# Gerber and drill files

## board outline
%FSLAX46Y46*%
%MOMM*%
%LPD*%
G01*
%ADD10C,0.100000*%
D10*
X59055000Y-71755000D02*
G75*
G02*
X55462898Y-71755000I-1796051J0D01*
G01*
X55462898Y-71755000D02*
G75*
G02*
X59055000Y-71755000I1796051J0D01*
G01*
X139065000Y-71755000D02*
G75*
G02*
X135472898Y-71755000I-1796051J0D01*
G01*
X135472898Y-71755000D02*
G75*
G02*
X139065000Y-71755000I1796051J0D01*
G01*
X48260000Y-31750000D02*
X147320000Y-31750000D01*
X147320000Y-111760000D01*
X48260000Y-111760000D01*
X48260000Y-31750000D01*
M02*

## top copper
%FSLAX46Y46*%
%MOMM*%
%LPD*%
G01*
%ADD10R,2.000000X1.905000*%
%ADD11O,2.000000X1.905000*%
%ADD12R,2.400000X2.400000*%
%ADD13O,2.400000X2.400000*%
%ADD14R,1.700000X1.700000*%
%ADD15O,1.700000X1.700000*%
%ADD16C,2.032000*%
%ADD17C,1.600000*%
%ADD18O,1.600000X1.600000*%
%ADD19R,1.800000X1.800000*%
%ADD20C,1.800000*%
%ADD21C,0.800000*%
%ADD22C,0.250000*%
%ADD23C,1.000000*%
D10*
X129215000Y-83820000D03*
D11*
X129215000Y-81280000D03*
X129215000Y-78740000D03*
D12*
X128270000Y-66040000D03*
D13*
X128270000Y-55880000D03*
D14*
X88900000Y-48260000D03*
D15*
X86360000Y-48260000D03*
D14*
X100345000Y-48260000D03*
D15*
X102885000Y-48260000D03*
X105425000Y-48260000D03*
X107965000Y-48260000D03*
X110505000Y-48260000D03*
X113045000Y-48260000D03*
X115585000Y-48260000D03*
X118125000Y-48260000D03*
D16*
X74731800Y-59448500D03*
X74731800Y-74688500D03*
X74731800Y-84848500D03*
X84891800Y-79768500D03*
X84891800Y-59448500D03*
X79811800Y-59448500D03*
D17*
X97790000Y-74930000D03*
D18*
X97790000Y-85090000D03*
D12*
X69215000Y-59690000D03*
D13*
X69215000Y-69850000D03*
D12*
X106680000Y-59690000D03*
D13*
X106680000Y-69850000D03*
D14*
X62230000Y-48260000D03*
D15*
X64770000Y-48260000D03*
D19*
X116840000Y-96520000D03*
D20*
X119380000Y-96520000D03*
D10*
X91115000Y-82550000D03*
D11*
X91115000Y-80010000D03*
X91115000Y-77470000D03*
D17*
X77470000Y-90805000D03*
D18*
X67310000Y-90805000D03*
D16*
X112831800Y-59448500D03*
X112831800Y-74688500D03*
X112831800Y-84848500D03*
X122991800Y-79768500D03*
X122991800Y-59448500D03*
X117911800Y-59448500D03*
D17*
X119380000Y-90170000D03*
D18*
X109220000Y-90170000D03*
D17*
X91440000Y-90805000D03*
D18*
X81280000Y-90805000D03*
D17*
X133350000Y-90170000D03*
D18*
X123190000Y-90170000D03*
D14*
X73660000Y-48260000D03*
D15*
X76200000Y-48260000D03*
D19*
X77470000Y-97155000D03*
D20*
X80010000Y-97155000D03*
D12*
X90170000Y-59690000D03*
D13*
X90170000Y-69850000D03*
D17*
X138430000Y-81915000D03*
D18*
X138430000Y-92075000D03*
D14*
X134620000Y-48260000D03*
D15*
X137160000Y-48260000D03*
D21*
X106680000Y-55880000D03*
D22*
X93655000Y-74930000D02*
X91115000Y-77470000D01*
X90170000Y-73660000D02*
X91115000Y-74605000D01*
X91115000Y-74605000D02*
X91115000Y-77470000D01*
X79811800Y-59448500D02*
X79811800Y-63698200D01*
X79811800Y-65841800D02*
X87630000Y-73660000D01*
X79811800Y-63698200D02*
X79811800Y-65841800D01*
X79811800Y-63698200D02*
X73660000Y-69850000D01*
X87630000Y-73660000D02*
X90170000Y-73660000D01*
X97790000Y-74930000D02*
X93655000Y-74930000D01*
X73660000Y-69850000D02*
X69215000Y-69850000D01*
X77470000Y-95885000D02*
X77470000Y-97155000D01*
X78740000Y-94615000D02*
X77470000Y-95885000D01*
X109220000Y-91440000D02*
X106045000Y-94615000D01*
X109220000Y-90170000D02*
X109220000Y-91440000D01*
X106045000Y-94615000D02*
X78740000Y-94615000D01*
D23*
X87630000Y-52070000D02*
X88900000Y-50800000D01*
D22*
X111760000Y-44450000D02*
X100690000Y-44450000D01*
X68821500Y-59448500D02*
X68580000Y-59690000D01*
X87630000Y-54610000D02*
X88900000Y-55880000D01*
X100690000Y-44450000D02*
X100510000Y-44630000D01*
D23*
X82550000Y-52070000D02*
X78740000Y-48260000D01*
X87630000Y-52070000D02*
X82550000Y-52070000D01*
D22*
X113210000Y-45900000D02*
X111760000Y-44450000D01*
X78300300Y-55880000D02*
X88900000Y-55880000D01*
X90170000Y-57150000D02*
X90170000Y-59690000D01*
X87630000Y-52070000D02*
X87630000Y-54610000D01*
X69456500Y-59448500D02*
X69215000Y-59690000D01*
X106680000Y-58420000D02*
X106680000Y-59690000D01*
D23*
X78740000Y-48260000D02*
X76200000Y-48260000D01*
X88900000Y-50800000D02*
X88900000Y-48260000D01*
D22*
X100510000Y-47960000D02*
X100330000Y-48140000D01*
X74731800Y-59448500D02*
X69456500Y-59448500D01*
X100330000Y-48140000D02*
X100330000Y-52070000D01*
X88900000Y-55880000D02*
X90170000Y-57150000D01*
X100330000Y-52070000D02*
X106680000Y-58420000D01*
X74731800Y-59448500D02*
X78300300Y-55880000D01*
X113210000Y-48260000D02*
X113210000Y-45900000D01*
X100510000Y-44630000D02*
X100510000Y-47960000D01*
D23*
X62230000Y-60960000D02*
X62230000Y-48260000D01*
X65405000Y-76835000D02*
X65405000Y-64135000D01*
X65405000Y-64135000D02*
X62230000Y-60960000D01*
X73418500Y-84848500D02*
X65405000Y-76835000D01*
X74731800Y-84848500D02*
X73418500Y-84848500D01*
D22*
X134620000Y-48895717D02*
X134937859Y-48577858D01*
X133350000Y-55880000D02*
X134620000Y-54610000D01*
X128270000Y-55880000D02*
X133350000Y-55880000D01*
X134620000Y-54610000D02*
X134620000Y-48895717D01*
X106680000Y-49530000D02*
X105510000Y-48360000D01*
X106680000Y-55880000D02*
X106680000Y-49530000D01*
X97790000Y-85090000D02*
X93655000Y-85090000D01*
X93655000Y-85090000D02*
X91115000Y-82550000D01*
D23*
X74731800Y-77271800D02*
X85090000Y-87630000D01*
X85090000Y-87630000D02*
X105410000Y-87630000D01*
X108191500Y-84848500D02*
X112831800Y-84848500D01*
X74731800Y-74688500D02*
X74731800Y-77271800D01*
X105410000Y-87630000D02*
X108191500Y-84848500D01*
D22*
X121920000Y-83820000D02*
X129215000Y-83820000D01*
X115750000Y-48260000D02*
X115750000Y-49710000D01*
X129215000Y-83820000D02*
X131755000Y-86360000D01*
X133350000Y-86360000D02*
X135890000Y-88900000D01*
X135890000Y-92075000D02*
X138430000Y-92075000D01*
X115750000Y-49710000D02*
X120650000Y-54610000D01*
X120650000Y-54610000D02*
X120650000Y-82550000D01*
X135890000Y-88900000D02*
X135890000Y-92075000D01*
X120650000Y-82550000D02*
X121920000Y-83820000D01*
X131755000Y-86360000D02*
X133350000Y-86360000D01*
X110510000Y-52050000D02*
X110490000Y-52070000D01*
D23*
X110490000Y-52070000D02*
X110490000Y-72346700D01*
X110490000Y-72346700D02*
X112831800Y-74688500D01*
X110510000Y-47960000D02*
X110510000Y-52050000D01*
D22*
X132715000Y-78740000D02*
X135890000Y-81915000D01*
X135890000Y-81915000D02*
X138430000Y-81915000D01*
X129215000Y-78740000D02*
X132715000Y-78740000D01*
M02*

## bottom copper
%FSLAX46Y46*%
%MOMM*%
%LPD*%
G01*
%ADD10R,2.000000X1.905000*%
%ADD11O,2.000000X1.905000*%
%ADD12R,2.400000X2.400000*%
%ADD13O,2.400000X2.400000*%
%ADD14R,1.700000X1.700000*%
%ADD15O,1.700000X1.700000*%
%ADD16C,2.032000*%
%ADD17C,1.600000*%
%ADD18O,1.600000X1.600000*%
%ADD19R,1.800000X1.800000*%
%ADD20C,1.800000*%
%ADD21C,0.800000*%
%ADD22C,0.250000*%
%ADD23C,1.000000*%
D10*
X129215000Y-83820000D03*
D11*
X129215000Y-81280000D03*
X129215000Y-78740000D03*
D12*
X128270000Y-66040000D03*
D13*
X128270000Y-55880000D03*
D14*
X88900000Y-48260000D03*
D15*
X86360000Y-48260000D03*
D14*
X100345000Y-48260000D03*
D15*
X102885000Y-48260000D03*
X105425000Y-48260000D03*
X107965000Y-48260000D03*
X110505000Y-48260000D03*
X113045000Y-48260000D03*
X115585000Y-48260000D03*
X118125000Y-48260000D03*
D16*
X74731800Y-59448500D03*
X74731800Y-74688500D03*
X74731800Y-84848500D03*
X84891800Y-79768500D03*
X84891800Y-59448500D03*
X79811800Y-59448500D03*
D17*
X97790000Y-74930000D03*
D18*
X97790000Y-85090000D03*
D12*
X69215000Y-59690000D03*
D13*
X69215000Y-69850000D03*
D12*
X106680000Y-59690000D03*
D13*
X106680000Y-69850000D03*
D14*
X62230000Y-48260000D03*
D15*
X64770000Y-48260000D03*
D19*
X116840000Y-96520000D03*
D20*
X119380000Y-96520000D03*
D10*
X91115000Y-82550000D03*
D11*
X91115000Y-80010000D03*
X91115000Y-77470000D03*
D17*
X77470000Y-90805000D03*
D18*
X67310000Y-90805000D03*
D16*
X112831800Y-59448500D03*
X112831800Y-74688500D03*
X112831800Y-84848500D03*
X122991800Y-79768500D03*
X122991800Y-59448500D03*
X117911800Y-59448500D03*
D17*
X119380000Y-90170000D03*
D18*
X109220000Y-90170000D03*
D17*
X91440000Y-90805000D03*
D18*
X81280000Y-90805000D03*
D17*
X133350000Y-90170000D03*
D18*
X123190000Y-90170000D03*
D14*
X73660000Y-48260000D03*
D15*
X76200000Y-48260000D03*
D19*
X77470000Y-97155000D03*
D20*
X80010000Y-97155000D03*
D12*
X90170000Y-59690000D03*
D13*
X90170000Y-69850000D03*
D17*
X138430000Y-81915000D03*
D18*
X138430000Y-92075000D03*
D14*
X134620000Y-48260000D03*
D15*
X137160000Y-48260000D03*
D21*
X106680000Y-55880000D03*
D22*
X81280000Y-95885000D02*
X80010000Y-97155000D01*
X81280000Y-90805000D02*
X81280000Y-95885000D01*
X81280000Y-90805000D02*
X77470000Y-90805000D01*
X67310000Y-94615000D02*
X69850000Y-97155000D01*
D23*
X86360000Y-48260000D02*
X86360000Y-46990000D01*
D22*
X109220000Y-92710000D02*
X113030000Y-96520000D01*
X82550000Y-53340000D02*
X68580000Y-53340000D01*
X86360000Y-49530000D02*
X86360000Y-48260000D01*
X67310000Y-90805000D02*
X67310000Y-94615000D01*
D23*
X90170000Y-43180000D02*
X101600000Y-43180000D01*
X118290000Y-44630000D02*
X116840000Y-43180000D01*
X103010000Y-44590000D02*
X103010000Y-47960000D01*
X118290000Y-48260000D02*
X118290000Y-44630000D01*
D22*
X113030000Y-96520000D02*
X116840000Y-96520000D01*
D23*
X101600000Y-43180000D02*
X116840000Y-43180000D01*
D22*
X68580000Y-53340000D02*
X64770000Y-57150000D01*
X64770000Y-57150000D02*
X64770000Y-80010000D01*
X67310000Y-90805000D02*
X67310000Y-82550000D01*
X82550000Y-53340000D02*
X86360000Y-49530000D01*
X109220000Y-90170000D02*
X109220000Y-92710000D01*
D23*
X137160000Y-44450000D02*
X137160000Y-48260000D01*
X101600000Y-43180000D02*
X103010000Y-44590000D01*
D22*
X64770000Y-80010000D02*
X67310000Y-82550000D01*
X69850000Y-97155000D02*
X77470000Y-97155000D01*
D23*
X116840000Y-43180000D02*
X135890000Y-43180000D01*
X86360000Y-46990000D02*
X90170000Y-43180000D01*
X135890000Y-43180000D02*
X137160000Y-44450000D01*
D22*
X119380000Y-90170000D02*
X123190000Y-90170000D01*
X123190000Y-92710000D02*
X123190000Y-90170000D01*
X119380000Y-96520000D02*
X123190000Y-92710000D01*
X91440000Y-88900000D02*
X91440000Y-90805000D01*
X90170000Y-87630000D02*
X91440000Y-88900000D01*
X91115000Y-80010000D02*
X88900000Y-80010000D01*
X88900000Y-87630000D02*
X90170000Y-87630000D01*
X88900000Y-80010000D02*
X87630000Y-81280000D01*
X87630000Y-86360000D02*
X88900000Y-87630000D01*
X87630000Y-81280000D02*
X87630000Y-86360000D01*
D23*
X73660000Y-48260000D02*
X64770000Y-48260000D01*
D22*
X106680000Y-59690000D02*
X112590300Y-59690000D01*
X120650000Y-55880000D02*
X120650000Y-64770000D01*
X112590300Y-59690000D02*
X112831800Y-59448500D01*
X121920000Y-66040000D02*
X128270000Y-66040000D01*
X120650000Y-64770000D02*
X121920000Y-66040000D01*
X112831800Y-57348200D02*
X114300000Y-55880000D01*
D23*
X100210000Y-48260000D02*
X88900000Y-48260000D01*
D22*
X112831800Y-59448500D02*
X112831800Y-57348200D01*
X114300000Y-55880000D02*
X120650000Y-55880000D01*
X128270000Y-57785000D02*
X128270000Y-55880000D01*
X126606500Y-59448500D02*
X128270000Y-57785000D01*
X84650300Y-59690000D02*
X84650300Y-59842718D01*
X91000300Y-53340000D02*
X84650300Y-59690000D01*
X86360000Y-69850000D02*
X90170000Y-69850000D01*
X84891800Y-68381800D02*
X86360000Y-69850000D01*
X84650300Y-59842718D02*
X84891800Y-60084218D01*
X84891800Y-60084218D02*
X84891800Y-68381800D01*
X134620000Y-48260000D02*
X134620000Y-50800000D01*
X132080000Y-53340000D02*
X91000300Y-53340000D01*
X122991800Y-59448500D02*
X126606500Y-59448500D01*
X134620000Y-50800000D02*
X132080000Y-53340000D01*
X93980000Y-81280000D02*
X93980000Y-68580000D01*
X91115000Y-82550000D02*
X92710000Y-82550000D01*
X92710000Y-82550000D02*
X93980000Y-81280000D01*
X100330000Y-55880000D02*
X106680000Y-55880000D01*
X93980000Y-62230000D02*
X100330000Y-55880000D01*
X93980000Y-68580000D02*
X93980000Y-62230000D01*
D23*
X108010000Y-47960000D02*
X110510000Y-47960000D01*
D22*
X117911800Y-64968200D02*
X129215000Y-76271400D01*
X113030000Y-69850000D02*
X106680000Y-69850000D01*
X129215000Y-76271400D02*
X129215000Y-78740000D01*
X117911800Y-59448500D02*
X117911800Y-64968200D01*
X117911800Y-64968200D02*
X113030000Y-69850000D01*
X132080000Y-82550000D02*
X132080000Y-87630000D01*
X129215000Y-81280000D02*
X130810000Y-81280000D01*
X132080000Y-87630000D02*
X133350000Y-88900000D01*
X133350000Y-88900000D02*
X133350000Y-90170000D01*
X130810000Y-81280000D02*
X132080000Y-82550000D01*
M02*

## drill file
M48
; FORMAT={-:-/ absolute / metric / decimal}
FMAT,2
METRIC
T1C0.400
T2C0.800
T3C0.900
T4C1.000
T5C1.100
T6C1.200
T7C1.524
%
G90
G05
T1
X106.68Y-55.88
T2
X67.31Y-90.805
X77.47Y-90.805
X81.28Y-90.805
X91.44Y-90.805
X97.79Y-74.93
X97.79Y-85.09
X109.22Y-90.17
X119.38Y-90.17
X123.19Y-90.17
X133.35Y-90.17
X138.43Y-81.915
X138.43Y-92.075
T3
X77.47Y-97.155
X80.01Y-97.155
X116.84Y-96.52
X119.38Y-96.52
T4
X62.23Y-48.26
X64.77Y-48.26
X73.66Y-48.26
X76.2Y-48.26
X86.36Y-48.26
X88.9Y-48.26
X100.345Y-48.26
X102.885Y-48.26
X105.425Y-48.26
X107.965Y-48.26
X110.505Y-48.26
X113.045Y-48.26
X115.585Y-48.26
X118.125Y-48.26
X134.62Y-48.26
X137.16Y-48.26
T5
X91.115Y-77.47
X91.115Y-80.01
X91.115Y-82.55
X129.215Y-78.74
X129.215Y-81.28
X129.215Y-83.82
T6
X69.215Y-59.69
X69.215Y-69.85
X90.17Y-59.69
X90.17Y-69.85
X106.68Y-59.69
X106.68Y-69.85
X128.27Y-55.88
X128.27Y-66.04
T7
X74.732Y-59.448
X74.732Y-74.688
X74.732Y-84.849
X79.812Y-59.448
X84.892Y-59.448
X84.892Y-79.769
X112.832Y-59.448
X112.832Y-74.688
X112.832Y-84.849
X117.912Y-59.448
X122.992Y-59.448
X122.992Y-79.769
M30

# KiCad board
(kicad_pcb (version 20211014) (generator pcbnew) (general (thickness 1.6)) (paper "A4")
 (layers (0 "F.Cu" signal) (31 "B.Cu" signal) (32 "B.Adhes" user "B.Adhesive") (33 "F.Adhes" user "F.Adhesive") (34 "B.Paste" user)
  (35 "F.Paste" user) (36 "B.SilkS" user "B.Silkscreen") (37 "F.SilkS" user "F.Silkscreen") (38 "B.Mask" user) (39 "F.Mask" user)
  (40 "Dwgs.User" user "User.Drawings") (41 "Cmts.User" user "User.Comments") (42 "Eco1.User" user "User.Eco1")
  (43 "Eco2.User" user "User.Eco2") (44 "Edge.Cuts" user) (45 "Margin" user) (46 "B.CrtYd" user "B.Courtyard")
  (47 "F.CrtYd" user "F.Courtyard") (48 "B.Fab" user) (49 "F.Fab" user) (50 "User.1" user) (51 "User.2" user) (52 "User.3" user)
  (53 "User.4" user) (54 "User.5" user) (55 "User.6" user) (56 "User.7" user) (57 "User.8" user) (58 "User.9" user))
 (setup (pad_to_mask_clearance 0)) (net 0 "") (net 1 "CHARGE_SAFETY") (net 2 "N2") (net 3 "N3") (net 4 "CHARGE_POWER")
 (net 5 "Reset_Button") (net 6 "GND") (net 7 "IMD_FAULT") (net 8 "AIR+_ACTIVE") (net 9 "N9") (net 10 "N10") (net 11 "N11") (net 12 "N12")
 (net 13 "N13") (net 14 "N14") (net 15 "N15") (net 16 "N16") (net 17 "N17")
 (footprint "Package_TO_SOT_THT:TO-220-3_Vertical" (layer "F.Cu") (at 129.215 83.82 90)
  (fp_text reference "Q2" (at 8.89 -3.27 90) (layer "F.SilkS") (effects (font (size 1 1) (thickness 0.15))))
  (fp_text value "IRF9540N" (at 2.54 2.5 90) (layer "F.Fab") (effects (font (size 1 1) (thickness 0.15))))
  (pad "1" thru_hole rect (at 0 0 90) (size 1.905 2) (drill 1.1) (layers *.Cu *.Mask) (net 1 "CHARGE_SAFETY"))
  (pad "2" thru_hole oval (at 2.54 0 90) (size 1.905 2) (drill 1.1) (layers *.Cu *.Mask) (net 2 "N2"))
  (pad "3" thru_hole oval (at 5.08 0 90) (size 1.905 2) (drill 1.1) (layers *.Cu *.Mask) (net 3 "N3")))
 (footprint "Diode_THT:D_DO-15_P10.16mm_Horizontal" (layer "F.Cu") (at 128.27 66.04 90)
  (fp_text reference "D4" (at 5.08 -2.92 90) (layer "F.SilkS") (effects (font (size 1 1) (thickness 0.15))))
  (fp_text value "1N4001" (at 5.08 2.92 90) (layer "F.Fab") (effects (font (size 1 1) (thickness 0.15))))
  (pad "1" thru_hole rect (at 0 0 90) (size 2.4 2.4) (drill 1.2) (layers *.Cu *.Mask) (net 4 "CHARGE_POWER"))
  (pad "2" thru_hole oval (at 10.16 0 90) (size 2.4 2.4) (drill 1.2) (layers *.Cu *.Mask) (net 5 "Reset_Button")))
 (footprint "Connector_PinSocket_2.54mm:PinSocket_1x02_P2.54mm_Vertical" (layer "F.Cu") (at 88.9 48.26 -90)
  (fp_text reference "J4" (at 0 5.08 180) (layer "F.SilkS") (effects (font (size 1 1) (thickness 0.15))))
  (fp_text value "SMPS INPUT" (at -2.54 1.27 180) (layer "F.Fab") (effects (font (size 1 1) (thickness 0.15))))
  (pad "1" thru_hole rect (at 0 0 270) (size 1.7 1.7) (drill 1) (layers *.Cu *.Mask) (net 4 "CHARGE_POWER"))
  (pad "2" thru_hole oval (at 0 2.54 270) (size 1.7 1.7) (drill 1) (layers *.Cu *.Mask) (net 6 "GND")))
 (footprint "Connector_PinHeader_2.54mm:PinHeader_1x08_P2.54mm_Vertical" (layer "F.Cu") (at 100.345 48.26 90)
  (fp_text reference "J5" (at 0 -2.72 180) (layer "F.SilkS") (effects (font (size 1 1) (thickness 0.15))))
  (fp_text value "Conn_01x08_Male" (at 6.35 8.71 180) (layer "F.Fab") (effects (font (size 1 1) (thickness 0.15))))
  (pad "1" thru_hole rect (at 0 0 90) (size 1.7 1.7) (drill 1) (layers *.Cu *.Mask) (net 4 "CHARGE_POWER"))
  (pad "2" thru_hole oval (at 0 2.54 90) (size 1.7 1.7) (drill 1) (layers *.Cu *.Mask) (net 6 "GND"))
  (pad "3" thru_hole oval (at 0 5.08 90) (size 1.7 1.7) (drill 1) (layers *.Cu *.Mask) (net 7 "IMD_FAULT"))
  (pad "4" thru_hole oval (at 0 7.62 90) (size 1.7 1.7) (drill 1) (layers *.Cu *.Mask) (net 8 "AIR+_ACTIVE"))
  (pad "5" thru_hole oval (at 0 10.16 90) (size 1.7 1.7) (drill 1) (layers *.Cu *.Mask) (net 8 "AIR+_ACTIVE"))
  (pad "6" thru_hole oval (at 0 12.7 90) (size 1.7 1.7) (drill 1) (layers *.Cu *.Mask) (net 4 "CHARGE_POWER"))
  (pad "7" thru_hole oval (at 0 15.24 90) (size 1.7 1.7) (drill 1) (layers *.Cu *.Mask) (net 1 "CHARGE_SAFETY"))
  (pad "8" thru_hole oval (at 0 17.78 90) (size 1.7 1.7) (drill 1) (layers *.Cu *.Mask) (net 6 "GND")))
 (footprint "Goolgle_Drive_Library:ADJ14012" (layer "F.Cu") (at 74.7318 59.4485)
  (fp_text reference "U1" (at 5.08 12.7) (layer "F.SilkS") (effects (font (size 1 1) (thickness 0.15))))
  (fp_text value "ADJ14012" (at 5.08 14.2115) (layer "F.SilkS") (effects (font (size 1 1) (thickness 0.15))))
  (pad "1" thru_hole circle locked (at 0 0) (size 2.032 2.032) (drill 1.524) (layers *.Cu *.Mask) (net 4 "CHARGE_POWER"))
  (pad "2" thru_hole circle locked (at 0 15.24) (size 2.032 2.032) (drill 1.524) (layers *.Cu *.Mask) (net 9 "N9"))
  (pad "4" thru_hole circle locked (at 0 25.4) (size 2.032 2.032) (drill 1.524) (layers *.Cu *.Mask) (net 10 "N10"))
  (pad "6" thru_hole circle locked (at 10.16 20.32) (size 2.032 2.032) (drill 1.524) (layers *.Cu *.Mask) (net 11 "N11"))
  (pad "8" thru_hole circle locked (at 10.16 0) (size 2.032 2.032) (drill 1.524) (layers *.Cu *.Mask) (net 5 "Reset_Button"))
  (pad "9" thru_hole circle locked (at 5.08 0) (size 2.032 2.032) (drill 1.524) (layers *.Cu *.Mask) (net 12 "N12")))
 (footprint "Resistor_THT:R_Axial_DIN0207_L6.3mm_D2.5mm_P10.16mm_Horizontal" (layer "F.Cu") (at 97.79 74.93 -90)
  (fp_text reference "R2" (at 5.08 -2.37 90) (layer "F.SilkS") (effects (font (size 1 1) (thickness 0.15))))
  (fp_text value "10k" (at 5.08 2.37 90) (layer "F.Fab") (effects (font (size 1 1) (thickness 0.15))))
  (pad "1" thru_hole circle (at 0 0 270) (size 1.6 1.6) (drill 0.8) (layers *.Cu *.Mask) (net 12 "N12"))
  (pad "2" thru_hole oval (at 10.16 0 270) (size 1.6 1.6) (drill 0.8) (layers *.Cu *.Mask) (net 7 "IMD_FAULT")))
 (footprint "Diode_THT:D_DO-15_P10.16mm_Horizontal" (layer "F.Cu") (at 69.215 59.69 -90)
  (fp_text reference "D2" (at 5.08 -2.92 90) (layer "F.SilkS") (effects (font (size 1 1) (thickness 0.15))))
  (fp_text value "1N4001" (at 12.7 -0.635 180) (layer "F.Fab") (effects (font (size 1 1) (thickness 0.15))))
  (pad "1" thru_hole rect (at 0 0 270) (size 2.4 2.4) (drill 1.2) (layers *.Cu *.Mask) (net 4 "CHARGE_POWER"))
  (pad "2" thru_hole oval (at 10.16 0 270) (size 2.4 2.4) (drill 1.2) (layers *.Cu *.Mask) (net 12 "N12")))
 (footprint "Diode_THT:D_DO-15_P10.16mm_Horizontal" (layer "F.Cu") (at 106.68 59.69 -90)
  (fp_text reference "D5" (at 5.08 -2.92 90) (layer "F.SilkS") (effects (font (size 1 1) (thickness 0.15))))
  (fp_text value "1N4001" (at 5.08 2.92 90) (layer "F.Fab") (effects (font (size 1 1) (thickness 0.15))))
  (pad "1" thru_hole rect (at 0 0 270) (size 2.4 2.4) (drill 1.2) (layers *.Cu *.Mask) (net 4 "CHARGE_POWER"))
  (pad "2" thru_hole oval (at 10.16 0 270) (size 2.4 2.4) (drill 1.2) (layers *.Cu *.Mask) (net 3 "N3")))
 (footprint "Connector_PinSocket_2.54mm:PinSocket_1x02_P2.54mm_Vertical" (layer "F.Cu") (at 62.23 48.26 90)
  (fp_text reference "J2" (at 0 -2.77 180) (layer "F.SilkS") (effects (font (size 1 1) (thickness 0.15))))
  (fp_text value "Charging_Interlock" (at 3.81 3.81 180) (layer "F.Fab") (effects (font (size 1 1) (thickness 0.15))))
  (pad "1" thru_hole rect (at 0 0 90) (size 1.7 1.7) (drill 1) (layers *.Cu *.Mask) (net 10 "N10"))
  (pad "2" thru_hole oval (at 0 2.54 90) (size 1.7 1.7) (drill 1) (layers *.Cu *.Mask) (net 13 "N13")))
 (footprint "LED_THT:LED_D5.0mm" (layer "F.Cu") (at 116.84 96.52)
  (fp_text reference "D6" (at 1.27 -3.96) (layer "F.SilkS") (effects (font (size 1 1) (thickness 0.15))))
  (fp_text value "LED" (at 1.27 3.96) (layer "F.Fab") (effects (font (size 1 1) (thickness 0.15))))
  (pad "1" thru_hole rect (at 0 0) (size 1.8 1.8) (drill 0.9) (layers *.Cu *.Mask) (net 6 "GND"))
  (pad "2" thru_hole circle (at 2.54 0) (size 1.8 1.8) (drill 0.9) (layers *.Cu *.Mask) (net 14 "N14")))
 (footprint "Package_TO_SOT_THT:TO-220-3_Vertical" (layer "F.Cu") (at 91.115 82.55 90)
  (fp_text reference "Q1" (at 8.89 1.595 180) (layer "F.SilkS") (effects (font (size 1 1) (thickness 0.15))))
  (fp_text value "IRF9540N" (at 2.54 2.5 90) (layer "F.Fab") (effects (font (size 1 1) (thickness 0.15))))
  (pad "1" thru_hole rect (at 0 0 90) (size 1.905 2) (drill 1.1) (layers *.Cu *.Mask) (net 7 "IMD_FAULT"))
  (pad "2" thru_hole oval (at 2.54 0 90) (size 1.905 2) (drill 1.1) (layers *.Cu *.Mask) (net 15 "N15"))
  (pad "3" thru_hole oval (at 5.08 0 90) (size 1.905 2) (drill 1.1) (layers *.Cu *.Mask) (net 12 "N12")))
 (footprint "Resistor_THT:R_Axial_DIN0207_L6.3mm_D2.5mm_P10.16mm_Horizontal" (layer "F.Cu") (at 77.47 90.805 180)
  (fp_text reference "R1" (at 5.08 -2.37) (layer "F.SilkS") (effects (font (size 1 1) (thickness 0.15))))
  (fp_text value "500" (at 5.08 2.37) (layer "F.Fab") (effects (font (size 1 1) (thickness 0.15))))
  (pad "1" thru_hole circle (at 0 0 180) (size 1.6 1.6) (drill 0.8) (layers *.Cu *.Mask) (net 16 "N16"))
  (pad "2" thru_hole oval (at 10.16 0 180) (size 1.6 1.6) (drill 0.8) (layers *.Cu *.Mask) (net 6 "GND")))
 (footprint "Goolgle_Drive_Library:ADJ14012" (layer "F.Cu") (at 112.8318 59.4485)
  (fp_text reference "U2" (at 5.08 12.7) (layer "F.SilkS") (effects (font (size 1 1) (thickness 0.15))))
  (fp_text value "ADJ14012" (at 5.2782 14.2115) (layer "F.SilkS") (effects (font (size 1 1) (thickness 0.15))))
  (pad "1" thru_hole circle locked (at 0 0) (size 2.032 2.032) (drill 1.524) (layers *.Cu *.Mask) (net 4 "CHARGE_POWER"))
  (pad "2" thru_hole circle locked (at 0 15.24) (size 2.032 2.032) (drill 1.524) (layers *.Cu *.Mask) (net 8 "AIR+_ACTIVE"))
  (pad "4" thru_hole circle locked (at 0 25.4) (size 2.032 2.032) (drill 1.524) (layers *.Cu *.Mask) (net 9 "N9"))
  (pad "6" thru_hole circle locked (at 10.16 20.32) (size 2.032 2.032) (drill 1.524) (layers *.Cu *.Mask) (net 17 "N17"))
  (pad "8" thru_hole circle locked (at 10.16 0) (size 2.032 2.032) (drill 1.524) (layers *.Cu *.Mask) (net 5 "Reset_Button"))
  (pad "9" thru_hole circle locked (at 5.08 0) (size 2.032 2.032) (drill 1.524) (layers *.Cu *.Mask) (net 3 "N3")))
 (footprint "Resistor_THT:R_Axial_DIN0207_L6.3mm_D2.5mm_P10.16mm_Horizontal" (layer "F.Cu") (at 119.38 90.17 180)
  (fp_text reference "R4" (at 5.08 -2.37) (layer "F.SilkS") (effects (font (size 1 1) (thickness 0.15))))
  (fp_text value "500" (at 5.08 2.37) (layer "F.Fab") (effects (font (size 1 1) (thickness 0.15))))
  (pad "1" thru_hole circle (at 0 0 180) (size 1.6 1.6) (drill 0.8) (layers *.Cu *.Mask) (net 14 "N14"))
  (pad "2" thru_hole oval (at 10.16 0 180) (size 1.6 1.6) (drill 0.8) (layers *.Cu *.Mask) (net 6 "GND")))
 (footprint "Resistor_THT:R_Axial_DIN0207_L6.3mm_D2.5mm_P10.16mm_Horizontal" (layer "F.Cu") (at 91.44 90.805 180)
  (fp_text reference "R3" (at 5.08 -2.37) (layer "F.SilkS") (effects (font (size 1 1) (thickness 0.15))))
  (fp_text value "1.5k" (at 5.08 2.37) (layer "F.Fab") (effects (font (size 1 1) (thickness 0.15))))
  (pad "1" thru_hole circle (at 0 0 180) (size 1.6 1.6) (drill 0.8) (layers *.Cu *.Mask) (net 15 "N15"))
  (pad "2" thru_hole oval (at 10.16 0 180) (size 1.6 1.6) (drill 0.8) (layers *.Cu *.Mask) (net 16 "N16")))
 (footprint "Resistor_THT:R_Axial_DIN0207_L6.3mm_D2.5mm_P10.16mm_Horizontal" (layer "F.Cu") (at 133.35 90.17 180)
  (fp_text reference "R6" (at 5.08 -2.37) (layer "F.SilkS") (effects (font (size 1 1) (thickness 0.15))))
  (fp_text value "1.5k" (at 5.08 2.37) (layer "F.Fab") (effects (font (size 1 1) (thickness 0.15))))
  (pad "1" thru_hole circle (at 0 0 180) (size 1.6 1.6) (drill 0.8) (layers *.Cu *.Mask) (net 2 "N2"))
  (pad "2" thru_hole oval (at 10.16 0 180) (size 1.6 1.6) (drill 0.8) (layers *.Cu *.Mask) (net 14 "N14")))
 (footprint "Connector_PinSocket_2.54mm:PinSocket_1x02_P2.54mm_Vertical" (layer "F.Cu") (at 73.66 48.26 90)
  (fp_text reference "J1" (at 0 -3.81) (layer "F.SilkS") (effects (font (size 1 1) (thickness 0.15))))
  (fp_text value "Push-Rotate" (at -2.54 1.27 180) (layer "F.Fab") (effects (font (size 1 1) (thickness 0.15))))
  (pad "1" thru_hole rect (at 0 0 90) (size 1.7 1.7) (drill 1) (layers *.Cu *.Mask) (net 13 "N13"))
  (pad "2" thru_hole oval (at 0 2.54 90) (size 1.7 1.7) (drill 1) (layers *.Cu *.Mask) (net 4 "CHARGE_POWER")))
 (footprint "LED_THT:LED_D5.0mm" (layer "F.Cu") (at 77.47 97.155)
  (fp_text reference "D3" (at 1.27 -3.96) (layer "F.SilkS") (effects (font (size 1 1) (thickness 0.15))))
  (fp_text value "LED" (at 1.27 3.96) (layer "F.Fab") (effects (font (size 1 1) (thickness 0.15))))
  (pad "1" thru_hole rect (at 0 0) (size 1.8 1.8) (drill 0.9) (layers *.Cu *.Mask) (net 6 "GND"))
  (pad "2" thru_hole circle (at 2.54 0) (size 1.8 1.8) (drill 0.9) (layers *.Cu *.Mask) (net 16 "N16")))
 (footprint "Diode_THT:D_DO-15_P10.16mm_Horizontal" (layer "F.Cu") (at 90.17 59.69 -90)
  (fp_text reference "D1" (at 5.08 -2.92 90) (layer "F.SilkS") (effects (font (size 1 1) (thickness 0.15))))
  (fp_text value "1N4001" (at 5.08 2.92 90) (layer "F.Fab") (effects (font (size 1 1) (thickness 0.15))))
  (pad "1" thru_hole rect (at 0 0 270) (size 2.4 2.4) (drill 1.2) (layers *.Cu *.Mask) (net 4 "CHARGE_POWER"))
  (pad "2" thru_hole oval (at 10.16 0 270) (size 2.4 2.4) (drill 1.2) (layers *.Cu *.Mask) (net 5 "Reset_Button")))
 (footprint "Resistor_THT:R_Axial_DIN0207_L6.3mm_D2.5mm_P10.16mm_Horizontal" (layer "F.Cu") (at 138.43 81.915 -90)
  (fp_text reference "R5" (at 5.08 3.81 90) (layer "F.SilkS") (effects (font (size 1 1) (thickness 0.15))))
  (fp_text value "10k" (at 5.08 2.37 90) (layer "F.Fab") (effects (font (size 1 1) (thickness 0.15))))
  (pad "1" thru_hole circle (at 0 0 270) (size 1.6 1.6) (drill 0.8) (layers *.Cu *.Mask) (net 3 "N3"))
  (pad "2" thru_hole oval (at 10.16 0 270) (size 1.6 1.6) (drill 0.8) (layers *.Cu *.Mask) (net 1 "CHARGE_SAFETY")))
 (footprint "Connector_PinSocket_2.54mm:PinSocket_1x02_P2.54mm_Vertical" (layer "F.Cu") (at 134.62 48.26 90)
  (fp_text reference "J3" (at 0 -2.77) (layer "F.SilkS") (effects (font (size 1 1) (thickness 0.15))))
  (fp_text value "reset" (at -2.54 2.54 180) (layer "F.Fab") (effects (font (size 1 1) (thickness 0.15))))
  (pad "1" thru_hole rect (at 0 0 90) (size 1.7 1.7) (drill 1) (layers *.Cu *.Mask) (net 5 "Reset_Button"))
  (pad "2" thru_hole oval (at 0 2.54 90) (size 1.7 1.7) (drill 1) (layers *.Cu *.Mask) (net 6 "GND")))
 (gr_circle (center 57.258949 71.755) (end 58.528949 73.025) (layer "Edge.Cuts") (width 0.1) (fill none))
 (gr_circle (center 137.268949 71.755) (end 135.998949 73.025) (layer "Edge.Cuts") (width 0.1) (fill none))
 (gr_rect (start 48.26 31.75) (end 147.32 111.76) (layer "Edge.Cuts") (width 0.1) (fill none))
 (segment (start 81.28 95.885) (end 80.01 97.155) (width 0.25) (layer "B.Cu") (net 16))
 (segment (start 81.28 90.805) (end 81.28 95.885) (width 0.25) (layer "B.Cu") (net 16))
 (segment (start 81.28 90.805) (end 77.47 90.805) (width 0.25) (layer "B.Cu") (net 16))
 (segment (start 93.655 74.93) (end 91.115 77.47) (width 0.25) (layer "F.Cu") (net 12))
 (segment (start 90.17 73.66) (end 91.115 74.605) (width 0.25) (layer "F.Cu") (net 12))
 (segment (start 91.115 74.605) (end 91.115 77.47) (width 0.25) (layer "F.Cu") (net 12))
 (segment (start 79.8118 59.4485) (end 79.8118 63.6982) (width 0.25) (layer "F.Cu") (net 12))
 (segment (start 79.8118 65.8418) (end 87.63 73.66) (width 0.25) (layer "F.Cu") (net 12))
 (segment (start 79.8118 63.6982) (end 79.8118 65.8418) (width 0.25) (layer "F.Cu") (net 12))
 (segment (start 79.8118 63.6982) (end 73.66 69.85) (width 0.25) (layer "F.Cu") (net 12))
 (segment (start 87.63 73.66) (end 90.17 73.66) (width 0.25) (layer "F.Cu") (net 12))
 (segment (start 97.79 74.93) (end 93.655 74.93) (width 0.25) (layer "F.Cu") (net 12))
 (segment (start 73.66 69.85) (end 69.215 69.85) (width 0.25) (layer "F.Cu") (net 12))
 (segment (start 77.47 95.885) (end 77.47 97.155) (width 0.25) (layer "F.Cu") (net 6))
 (segment (start 78.74 94.615) (end 77.47 95.885) (width 0.25) (layer "F.Cu") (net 6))
 (segment (start 109.22 91.44) (end 106.045 94.615) (width 0.25) (layer "F.Cu") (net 6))
 (segment (start 109.22 90.17) (end 109.22 91.44) (width 0.25) (layer "F.Cu") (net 6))
 (segment (start 106.045 94.615) (end 78.74 94.615) (width 0.25) (layer "F.Cu") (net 6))
 (segment (start 67.31 94.615) (end 69.85 97.155) (width 0.25) (layer "B.Cu") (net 6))
 (segment (start 86.36 48.26) (end 86.36 46.99) (width 1) (layer "B.Cu") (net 6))
 (segment (start 109.22 92.71) (end 113.03 96.52) (width 0.25) (layer "B.Cu") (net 6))
 (segment (start 82.55 53.34) (end 68.58 53.34) (width 0.25) (layer "B.Cu") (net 6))
 (segment (start 86.36 49.53) (end 86.36 48.26) (width 0.25) (layer "B.Cu") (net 6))
 (segment (start 67.31 90.805) (end 67.31 94.615) (width 0.25) (layer "B.Cu") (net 6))
 (segment (start 90.17 43.18) (end 101.6 43.18) (width 1) (layer "B.Cu") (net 6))
 (segment (start 118.29 44.63) (end 116.84 43.18) (width 1) (layer "B.Cu") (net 6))
 (segment (start 103.01 44.59) (end 103.01 47.96) (width 1) (layer "B.Cu") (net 6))
 (segment (start 118.29 48.26) (end 118.29 44.63) (width 1) (layer "B.Cu") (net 6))
 (segment (start 113.03 96.52) (end 116.84 96.52) (width 0.25) (layer "B.Cu") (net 6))
 (segment (start 101.6 43.18) (end 116.84 43.18) (width 1) (layer "B.Cu") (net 6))
 (segment (start 68.58 53.34) (end 64.77 57.15) (width 0.25) (layer "B.Cu") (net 6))
 (segment (start 64.77 57.15) (end 64.77 80.01) (width 0.25) (layer "B.Cu") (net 6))
 (segment (start 67.31 90.805) (end 67.31 82.55) (width 0.25) (layer "B.Cu") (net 6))
 (segment (start 82.55 53.34) (end 86.36 49.53) (width 0.25) (layer "B.Cu") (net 6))
 (segment (start 109.22 90.17) (end 109.22 92.71) (width 0.25) (layer "B.Cu") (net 6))
 (segment (start 137.16 44.45) (end 137.16 48.26) (width 1) (layer "B.Cu") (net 6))
 (segment (start 101.6 43.18) (end 103.01 44.59) (width 1) (layer "B.Cu") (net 6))
 (segment (start 64.77 80.01) (end 67.31 82.55) (width 0.25) (layer "B.Cu") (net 6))
 (segment (start 69.85 97.155) (end 77.47 97.155) (width 0.25) (layer "B.Cu") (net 6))
 (segment (start 116.84 43.18) (end 135.89 43.18) (width 1) (layer "B.Cu") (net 6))
 (segment (start 86.36 46.99) (end 90.17 43.18) (width 1) (layer "B.Cu") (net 6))
 (segment (start 135.89 43.18) (end 137.16 44.45) (width 1) (layer "B.Cu") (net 6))
 (segment (start 119.38 90.17) (end 123.19 90.17) (width 0.25) (layer "B.Cu") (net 14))
 (segment (start 123.19 92.71) (end 123.19 90.17) (width 0.25) (layer "B.Cu") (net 14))
 (segment (start 119.38 96.52) (end 123.19 92.71) (width 0.25) (layer "B.Cu") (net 14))
 (segment (start 91.44 88.9) (end 91.44 90.805) (width 0.25) (layer "B.Cu") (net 15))
 (segment (start 90.17 87.63) (end 91.44 88.9) (width 0.25) (layer "B.Cu") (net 15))
 (segment (start 91.115 80.01) (end 88.9 80.01) (width 0.25) (layer "B.Cu") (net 15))
 (segment (start 88.9 87.63) (end 90.17 87.63) (width 0.25) (layer "B.Cu") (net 15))
 (segment (start 88.9 80.01) (end 87.63 81.28) (width 0.25) (layer "B.Cu") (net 15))
 (segment (start 87.63 86.36) (end 88.9 87.63) (width 0.25) (layer "B.Cu") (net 15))
 (segment (start 87.63 81.28) (end 87.63 86.36) (width 0.25) (layer "B.Cu") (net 15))
 (segment (start 73.66 48.26) (end 64.77 48.26) (width 1) (layer "B.Cu") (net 13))
 (segment (start 87.63 52.07) (end 88.9 50.8) (width 1) (layer "F.Cu") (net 4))
 (segment (start 111.76 44.45) (end 100.69 44.45) (width 0.25) (layer "F.Cu") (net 4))
 (segment (start 68.8215 59.4485) (end 68.58 59.69) (width 0.25) (layer "F.Cu") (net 4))
 (segment (start 87.63 54.61) (end 88.9 55.88) (width 0.25) (layer "F.Cu") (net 4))
 (segment (start 100.69 44.45) (end 100.51 44.63) (width 0.25) (layer "F.Cu") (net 4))
 (segment (start 82.55 52.07) (end 78.74 48.26) (width 1) (layer "F.Cu") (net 4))
 (segment (start 87.63 52.07) (end 82.55 52.07) (width 1) (layer "F.Cu") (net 4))
 (segment (start 113.21 45.9) (end 111.76 44.45) (width 0.25) (layer "F.Cu") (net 4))
 (segment (start 78.3003 55.88) (end 88.9 55.88) (width 0.25) (layer "F.Cu") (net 4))
 (segment (start 90.17 57.15) (end 90.17 59.69) (width 0.25) (layer "F.Cu") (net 4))
 (segment (start 87.63 52.07) (end 87.63 54.61) (width 0.25) (layer "F.Cu") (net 4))
 (segment (start 69.4565 59.4485) (end 69.215 59.69) (width 0.25) (layer "F.Cu") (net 4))
 (segment (start 106.68 58.42) (end 106.68 59.69) (width 0.25) (layer "F.Cu") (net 4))
 (segment (start 78.74 48.26) (end 76.2 48.26) (width 1) (layer "F.Cu") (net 4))
 (segment (start 88.9 50.8) (end 88.9 48.26) (width 1) (layer "F.Cu") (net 4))
 (segment (start 100.51 47.96) (end 100.33 48.14) (width 0.25) (layer "F.Cu") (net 4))
 (segment (start 74.7318 59.4485) (end 69.4565 59.4485) (width 0.25) (layer "F.Cu") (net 4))
 (segment (start 100.33 48.14) (end 100.33 52.07) (width 0.25) (layer "F.Cu") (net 4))
 (segment (start 88.9 55.88) (end 90.17 57.15) (width 0.25) (layer "F.Cu") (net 4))
 (segment (start 100.33 52.07) (end 106.68 58.42) (width 0.25) (layer "F.Cu") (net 4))
 (segment (start 74.7318 59.4485) (end 78.3003 55.88) (width 0.25) (layer "F.Cu") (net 4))
 (segment (start 113.21 48.26) (end 113.21 45.9) (width 0.25) (layer "F.Cu") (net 4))
 (segment (start 100.51 44.63) (end 100.51 47.96) (width 0.25) (layer "F.Cu") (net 4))
 (segment (start 106.68 59.69) (end 112.5903 59.69) (width 0.25) (layer "B.Cu") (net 4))
 (segment (start 120.65 55.88) (end 120.65 64.77) (width 0.25) (layer "B.Cu") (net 4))
 (segment (start 112.5903 59.69) (end 112.8318 59.4485) (width 0.25) (layer "B.Cu") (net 4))
 (segment (start 121.92 66.04) (end 128.27 66.04) (width 0.25) (layer "B.Cu") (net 4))
 (segment (start 120.65 64.77) (end 121.92 66.04) (width 0.25) (layer "B.Cu") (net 4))
 (segment (start 112.8318 57.3482) (end 114.3 55.88) (width 0.25) (layer "B.Cu") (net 4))
 (segment (start 100.21 48.26) (end 88.9 48.26) (width 1) (layer "B.Cu") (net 4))
 (segment (start 112.8318 59.4485) (end 112.8318 57.3482) (width 0.25) (layer "B.Cu") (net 4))
 (segment (start 114.3 55.88) (end 120.65 55.88) (width 0.25) (layer "B.Cu") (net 4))
 (segment (start 62.23 60.96) (end 62.23 48.26) (width 1) (layer "F.Cu") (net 10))
 (segment (start 65.405 76.835) (end 65.405 64.135) (width 1) (layer "F.Cu") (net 10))
 (segment (start 65.405 64.135) (end 62.23 60.96) (width 1) (layer "F.Cu") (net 10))
 (segment (start 73.4185 84.8485) (end 65.405 76.835) (width 1) (layer "F.Cu") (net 10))
 (segment (start 74.7318 84.8485) (end 73.4185 84.8485) (width 1) (layer "F.Cu") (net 10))
 (segment (start 134.62 48.895717) (end 134.937859 48.577858) (width 0.25) (layer "F.Cu") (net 5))
 (segment (start 133.35 55.88) (end 134.62 54.61) (width 0.25) (layer "F.Cu") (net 5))
 (segment (start 128.27 55.88) (end 133.35 55.88) (width 0.25) (layer "F.Cu") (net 5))
 (segment (start 134.62 54.61) (end 134.62 48.895717) (width 0.25) (layer "F.Cu") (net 5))
 (segment (start 128.27 57.785) (end 128.27 55.88) (width 0.25) (layer "B.Cu") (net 5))
 (segment (start 126.6065 59.4485) (end 128.27 57.785) (width 0.25) (layer "B.Cu") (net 5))
 (segment (start 84.6503 59.69) (end 84.6503 59.842718) (width 0.25) (layer "B.Cu") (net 5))
 (segment (start 91.0003 53.34) (end 84.6503 59.69) (width 0.25) (layer "B.Cu") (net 5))
 (segment (start 86.36 69.85) (end 90.17 69.85) (width 0.25) (layer "B.Cu") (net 5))
 (segment (start 84.8918 68.3818) (end 86.36 69.85) (width 0.25) (layer "B.Cu") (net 5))
 (segment (start 84.6503 59.842718) (end 84.8918 60.084218) (width 0.25) (layer "B.Cu") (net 5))
 (segment (start 84.8918 60.084218) (end 84.8918 68.3818) (width 0.25) (layer "B.Cu") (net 5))
 (segment (start 134.62 48.26) (end 134.62 50.8) (width 0.25) (layer "B.Cu") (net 5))
 (segment (start 132.08 53.34) (end 91.0003 53.34) (width 0.25) (layer "B.Cu") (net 5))
 (segment (start 122.9918 59.4485) (end 126.6065 59.4485) (width 0.25) (layer "B.Cu") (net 5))
 (segment (start 134.62 50.8) (end 132.08 53.34) (width 0.25) (layer "B.Cu") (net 5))
 (segment (start 106.68 49.53) (end 105.51 48.36) (width 0.25) (layer "F.Cu") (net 7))
 (segment (start 106.68 55.88) (end 106.68 49.53) (width 0.25) (layer "F.Cu") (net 7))
 (segment (start 97.79 85.09) (end 93.655 85.09) (width 0.25) (layer "F.Cu") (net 7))
 (segment (start 93.655 85.09) (end 91.115 82.55) (width 0.25) (layer "F.Cu") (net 7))
 (via (at 106.68 55.88) (size 0.8) (drill 0.4) (layers "F.Cu" "B.Cu") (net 7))
 (segment (start 93.98 81.28) (end 93.98 68.58) (width 0.25) (layer "B.Cu") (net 7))
 (segment (start 91.115 82.55) (end 92.71 82.55) (width 0.25) (layer "B.Cu") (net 7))
 (segment (start 92.71 82.55) (end 93.98 81.28) (width 0.25) (layer "B.Cu") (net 7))
 (segment (start 100.33 55.88) (end 106.68 55.88) (width 0.25) (layer "B.Cu") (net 7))
 (segment (start 93.98 62.23) (end 100.33 55.88) (width 0.25) (layer "B.Cu") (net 7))
 (segment (start 93.98 68.58) (end 93.98 62.23) (width 0.25) (layer "B.Cu") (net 7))
 (segment (start 74.7318 77.2718) (end 85.09 87.63) (width 1) (layer "F.Cu") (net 9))
 (segment (start 85.09 87.63) (end 105.41 87.63) (width 1) (layer "F.Cu") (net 9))
 (segment (start 108.1915 84.8485) (end 112.8318 84.8485) (width 1) (layer "F.Cu") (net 9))
 (segment (start 74.7318 74.6885) (end 74.7318 77.2718) (width 1) (layer "F.Cu") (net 9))
 (segment (start 105.41 87.63) (end 108.1915 84.8485) (width 1) (layer "F.Cu") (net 9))
 (segment (start 121.92 83.82) (end 129.215 83.82) (width 0.25) (layer "F.Cu") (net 1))
 (segment (start 115.75 48.26) (end 115.75 49.71) (width 0.25) (layer "F.Cu") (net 1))
 (segment (start 129.215 83.82) (end 131.755 86.36) (width 0.25) (layer "F.Cu") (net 1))
 (segment (start 133.35 86.36) (end 135.89 88.9) (width 0.25) (layer "F.Cu") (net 1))
 (segment (start 135.89 92.075) (end 138.43 92.075) (width 0.25) (layer "F.Cu") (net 1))
 (segment (start 115.75 49.71) (end 120.65 54.61) (width 0.25) (layer "F.Cu") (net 1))
 (segment (start 120.65 54.61) (end 120.65 82.55) (width 0.25) (layer "F.Cu") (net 1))
 (segment (start 135.89 88.9) (end 135.89 92.075) (width 0.25) (layer "F.Cu") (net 1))
 (segment (start 120.65 82.55) (end 121.92 83.82) (width 0.25) (layer "F.Cu") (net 1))
 (segment (start 131.755 86.36) (end 133.35 86.36) (width 0.25) (layer "F.Cu") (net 1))
 (segment (start 110.51 52.05) (end 110.49 52.07) (width 0.25) (layer "F.Cu") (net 8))
 (segment (start 110.49 52.07) (end 110.49 72.3467) (width 1) (layer "F.Cu") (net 8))
 (segment (start 110.49 72.3467) (end 112.8318 74.6885) (width 1) (layer "F.Cu") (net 8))
 (segment (start 110.51 47.96) (end 110.51 52.05) (width 1) (layer "F.Cu") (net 8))
 (segment (start 108.01 47.96) (end 110.51 47.96) (width 1) (layer "B.Cu") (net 8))
 (segment (start 132.715 78.74) (end 135.89 81.915) (width 0.25) (layer "F.Cu") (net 3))
 (segment (start 135.89 81.915) (end 138.43 81.915) (width 0.25) (layer "F.Cu") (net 3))
 (segment (start 129.215 78.74) (end 132.715 78.74) (width 0.25) (layer "F.Cu") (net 3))
 (segment (start 117.9118 64.9682) (end 129.215 76.2714) (width 0.25) (layer "B.Cu") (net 3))
 (segment (start 113.03 69.85) (end 106.68 69.85) (width 0.25) (layer "B.Cu") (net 3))
 (segment (start 129.215 76.2714) (end 129.215 78.74) (width 0.25) (layer "B.Cu") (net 3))
 (segment (start 117.9118 59.4485) (end 117.9118 64.9682) (width 0.25) (layer "B.Cu") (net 3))
 (segment (start 117.9118 64.9682) (end 113.03 69.85) (width 0.25) (layer "B.Cu") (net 3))
 (segment (start 132.08 82.55) (end 132.08 87.63) (width 0.25) (layer "B.Cu") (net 2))
 (segment (start 129.215 81.28) (end 130.81 81.28) (width 0.25) (layer "B.Cu") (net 2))
 (segment (start 132.08 87.63) (end 133.35 88.9) (width 0.25) (layer "B.Cu") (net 2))
 (segment (start 133.35 88.9) (end 133.35 90.17) (width 0.25) (layer "B.Cu") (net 2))
 (segment (start 130.81 81.28) (end 132.08 82.55) (width 0.25) (layer "B.Cu") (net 2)))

